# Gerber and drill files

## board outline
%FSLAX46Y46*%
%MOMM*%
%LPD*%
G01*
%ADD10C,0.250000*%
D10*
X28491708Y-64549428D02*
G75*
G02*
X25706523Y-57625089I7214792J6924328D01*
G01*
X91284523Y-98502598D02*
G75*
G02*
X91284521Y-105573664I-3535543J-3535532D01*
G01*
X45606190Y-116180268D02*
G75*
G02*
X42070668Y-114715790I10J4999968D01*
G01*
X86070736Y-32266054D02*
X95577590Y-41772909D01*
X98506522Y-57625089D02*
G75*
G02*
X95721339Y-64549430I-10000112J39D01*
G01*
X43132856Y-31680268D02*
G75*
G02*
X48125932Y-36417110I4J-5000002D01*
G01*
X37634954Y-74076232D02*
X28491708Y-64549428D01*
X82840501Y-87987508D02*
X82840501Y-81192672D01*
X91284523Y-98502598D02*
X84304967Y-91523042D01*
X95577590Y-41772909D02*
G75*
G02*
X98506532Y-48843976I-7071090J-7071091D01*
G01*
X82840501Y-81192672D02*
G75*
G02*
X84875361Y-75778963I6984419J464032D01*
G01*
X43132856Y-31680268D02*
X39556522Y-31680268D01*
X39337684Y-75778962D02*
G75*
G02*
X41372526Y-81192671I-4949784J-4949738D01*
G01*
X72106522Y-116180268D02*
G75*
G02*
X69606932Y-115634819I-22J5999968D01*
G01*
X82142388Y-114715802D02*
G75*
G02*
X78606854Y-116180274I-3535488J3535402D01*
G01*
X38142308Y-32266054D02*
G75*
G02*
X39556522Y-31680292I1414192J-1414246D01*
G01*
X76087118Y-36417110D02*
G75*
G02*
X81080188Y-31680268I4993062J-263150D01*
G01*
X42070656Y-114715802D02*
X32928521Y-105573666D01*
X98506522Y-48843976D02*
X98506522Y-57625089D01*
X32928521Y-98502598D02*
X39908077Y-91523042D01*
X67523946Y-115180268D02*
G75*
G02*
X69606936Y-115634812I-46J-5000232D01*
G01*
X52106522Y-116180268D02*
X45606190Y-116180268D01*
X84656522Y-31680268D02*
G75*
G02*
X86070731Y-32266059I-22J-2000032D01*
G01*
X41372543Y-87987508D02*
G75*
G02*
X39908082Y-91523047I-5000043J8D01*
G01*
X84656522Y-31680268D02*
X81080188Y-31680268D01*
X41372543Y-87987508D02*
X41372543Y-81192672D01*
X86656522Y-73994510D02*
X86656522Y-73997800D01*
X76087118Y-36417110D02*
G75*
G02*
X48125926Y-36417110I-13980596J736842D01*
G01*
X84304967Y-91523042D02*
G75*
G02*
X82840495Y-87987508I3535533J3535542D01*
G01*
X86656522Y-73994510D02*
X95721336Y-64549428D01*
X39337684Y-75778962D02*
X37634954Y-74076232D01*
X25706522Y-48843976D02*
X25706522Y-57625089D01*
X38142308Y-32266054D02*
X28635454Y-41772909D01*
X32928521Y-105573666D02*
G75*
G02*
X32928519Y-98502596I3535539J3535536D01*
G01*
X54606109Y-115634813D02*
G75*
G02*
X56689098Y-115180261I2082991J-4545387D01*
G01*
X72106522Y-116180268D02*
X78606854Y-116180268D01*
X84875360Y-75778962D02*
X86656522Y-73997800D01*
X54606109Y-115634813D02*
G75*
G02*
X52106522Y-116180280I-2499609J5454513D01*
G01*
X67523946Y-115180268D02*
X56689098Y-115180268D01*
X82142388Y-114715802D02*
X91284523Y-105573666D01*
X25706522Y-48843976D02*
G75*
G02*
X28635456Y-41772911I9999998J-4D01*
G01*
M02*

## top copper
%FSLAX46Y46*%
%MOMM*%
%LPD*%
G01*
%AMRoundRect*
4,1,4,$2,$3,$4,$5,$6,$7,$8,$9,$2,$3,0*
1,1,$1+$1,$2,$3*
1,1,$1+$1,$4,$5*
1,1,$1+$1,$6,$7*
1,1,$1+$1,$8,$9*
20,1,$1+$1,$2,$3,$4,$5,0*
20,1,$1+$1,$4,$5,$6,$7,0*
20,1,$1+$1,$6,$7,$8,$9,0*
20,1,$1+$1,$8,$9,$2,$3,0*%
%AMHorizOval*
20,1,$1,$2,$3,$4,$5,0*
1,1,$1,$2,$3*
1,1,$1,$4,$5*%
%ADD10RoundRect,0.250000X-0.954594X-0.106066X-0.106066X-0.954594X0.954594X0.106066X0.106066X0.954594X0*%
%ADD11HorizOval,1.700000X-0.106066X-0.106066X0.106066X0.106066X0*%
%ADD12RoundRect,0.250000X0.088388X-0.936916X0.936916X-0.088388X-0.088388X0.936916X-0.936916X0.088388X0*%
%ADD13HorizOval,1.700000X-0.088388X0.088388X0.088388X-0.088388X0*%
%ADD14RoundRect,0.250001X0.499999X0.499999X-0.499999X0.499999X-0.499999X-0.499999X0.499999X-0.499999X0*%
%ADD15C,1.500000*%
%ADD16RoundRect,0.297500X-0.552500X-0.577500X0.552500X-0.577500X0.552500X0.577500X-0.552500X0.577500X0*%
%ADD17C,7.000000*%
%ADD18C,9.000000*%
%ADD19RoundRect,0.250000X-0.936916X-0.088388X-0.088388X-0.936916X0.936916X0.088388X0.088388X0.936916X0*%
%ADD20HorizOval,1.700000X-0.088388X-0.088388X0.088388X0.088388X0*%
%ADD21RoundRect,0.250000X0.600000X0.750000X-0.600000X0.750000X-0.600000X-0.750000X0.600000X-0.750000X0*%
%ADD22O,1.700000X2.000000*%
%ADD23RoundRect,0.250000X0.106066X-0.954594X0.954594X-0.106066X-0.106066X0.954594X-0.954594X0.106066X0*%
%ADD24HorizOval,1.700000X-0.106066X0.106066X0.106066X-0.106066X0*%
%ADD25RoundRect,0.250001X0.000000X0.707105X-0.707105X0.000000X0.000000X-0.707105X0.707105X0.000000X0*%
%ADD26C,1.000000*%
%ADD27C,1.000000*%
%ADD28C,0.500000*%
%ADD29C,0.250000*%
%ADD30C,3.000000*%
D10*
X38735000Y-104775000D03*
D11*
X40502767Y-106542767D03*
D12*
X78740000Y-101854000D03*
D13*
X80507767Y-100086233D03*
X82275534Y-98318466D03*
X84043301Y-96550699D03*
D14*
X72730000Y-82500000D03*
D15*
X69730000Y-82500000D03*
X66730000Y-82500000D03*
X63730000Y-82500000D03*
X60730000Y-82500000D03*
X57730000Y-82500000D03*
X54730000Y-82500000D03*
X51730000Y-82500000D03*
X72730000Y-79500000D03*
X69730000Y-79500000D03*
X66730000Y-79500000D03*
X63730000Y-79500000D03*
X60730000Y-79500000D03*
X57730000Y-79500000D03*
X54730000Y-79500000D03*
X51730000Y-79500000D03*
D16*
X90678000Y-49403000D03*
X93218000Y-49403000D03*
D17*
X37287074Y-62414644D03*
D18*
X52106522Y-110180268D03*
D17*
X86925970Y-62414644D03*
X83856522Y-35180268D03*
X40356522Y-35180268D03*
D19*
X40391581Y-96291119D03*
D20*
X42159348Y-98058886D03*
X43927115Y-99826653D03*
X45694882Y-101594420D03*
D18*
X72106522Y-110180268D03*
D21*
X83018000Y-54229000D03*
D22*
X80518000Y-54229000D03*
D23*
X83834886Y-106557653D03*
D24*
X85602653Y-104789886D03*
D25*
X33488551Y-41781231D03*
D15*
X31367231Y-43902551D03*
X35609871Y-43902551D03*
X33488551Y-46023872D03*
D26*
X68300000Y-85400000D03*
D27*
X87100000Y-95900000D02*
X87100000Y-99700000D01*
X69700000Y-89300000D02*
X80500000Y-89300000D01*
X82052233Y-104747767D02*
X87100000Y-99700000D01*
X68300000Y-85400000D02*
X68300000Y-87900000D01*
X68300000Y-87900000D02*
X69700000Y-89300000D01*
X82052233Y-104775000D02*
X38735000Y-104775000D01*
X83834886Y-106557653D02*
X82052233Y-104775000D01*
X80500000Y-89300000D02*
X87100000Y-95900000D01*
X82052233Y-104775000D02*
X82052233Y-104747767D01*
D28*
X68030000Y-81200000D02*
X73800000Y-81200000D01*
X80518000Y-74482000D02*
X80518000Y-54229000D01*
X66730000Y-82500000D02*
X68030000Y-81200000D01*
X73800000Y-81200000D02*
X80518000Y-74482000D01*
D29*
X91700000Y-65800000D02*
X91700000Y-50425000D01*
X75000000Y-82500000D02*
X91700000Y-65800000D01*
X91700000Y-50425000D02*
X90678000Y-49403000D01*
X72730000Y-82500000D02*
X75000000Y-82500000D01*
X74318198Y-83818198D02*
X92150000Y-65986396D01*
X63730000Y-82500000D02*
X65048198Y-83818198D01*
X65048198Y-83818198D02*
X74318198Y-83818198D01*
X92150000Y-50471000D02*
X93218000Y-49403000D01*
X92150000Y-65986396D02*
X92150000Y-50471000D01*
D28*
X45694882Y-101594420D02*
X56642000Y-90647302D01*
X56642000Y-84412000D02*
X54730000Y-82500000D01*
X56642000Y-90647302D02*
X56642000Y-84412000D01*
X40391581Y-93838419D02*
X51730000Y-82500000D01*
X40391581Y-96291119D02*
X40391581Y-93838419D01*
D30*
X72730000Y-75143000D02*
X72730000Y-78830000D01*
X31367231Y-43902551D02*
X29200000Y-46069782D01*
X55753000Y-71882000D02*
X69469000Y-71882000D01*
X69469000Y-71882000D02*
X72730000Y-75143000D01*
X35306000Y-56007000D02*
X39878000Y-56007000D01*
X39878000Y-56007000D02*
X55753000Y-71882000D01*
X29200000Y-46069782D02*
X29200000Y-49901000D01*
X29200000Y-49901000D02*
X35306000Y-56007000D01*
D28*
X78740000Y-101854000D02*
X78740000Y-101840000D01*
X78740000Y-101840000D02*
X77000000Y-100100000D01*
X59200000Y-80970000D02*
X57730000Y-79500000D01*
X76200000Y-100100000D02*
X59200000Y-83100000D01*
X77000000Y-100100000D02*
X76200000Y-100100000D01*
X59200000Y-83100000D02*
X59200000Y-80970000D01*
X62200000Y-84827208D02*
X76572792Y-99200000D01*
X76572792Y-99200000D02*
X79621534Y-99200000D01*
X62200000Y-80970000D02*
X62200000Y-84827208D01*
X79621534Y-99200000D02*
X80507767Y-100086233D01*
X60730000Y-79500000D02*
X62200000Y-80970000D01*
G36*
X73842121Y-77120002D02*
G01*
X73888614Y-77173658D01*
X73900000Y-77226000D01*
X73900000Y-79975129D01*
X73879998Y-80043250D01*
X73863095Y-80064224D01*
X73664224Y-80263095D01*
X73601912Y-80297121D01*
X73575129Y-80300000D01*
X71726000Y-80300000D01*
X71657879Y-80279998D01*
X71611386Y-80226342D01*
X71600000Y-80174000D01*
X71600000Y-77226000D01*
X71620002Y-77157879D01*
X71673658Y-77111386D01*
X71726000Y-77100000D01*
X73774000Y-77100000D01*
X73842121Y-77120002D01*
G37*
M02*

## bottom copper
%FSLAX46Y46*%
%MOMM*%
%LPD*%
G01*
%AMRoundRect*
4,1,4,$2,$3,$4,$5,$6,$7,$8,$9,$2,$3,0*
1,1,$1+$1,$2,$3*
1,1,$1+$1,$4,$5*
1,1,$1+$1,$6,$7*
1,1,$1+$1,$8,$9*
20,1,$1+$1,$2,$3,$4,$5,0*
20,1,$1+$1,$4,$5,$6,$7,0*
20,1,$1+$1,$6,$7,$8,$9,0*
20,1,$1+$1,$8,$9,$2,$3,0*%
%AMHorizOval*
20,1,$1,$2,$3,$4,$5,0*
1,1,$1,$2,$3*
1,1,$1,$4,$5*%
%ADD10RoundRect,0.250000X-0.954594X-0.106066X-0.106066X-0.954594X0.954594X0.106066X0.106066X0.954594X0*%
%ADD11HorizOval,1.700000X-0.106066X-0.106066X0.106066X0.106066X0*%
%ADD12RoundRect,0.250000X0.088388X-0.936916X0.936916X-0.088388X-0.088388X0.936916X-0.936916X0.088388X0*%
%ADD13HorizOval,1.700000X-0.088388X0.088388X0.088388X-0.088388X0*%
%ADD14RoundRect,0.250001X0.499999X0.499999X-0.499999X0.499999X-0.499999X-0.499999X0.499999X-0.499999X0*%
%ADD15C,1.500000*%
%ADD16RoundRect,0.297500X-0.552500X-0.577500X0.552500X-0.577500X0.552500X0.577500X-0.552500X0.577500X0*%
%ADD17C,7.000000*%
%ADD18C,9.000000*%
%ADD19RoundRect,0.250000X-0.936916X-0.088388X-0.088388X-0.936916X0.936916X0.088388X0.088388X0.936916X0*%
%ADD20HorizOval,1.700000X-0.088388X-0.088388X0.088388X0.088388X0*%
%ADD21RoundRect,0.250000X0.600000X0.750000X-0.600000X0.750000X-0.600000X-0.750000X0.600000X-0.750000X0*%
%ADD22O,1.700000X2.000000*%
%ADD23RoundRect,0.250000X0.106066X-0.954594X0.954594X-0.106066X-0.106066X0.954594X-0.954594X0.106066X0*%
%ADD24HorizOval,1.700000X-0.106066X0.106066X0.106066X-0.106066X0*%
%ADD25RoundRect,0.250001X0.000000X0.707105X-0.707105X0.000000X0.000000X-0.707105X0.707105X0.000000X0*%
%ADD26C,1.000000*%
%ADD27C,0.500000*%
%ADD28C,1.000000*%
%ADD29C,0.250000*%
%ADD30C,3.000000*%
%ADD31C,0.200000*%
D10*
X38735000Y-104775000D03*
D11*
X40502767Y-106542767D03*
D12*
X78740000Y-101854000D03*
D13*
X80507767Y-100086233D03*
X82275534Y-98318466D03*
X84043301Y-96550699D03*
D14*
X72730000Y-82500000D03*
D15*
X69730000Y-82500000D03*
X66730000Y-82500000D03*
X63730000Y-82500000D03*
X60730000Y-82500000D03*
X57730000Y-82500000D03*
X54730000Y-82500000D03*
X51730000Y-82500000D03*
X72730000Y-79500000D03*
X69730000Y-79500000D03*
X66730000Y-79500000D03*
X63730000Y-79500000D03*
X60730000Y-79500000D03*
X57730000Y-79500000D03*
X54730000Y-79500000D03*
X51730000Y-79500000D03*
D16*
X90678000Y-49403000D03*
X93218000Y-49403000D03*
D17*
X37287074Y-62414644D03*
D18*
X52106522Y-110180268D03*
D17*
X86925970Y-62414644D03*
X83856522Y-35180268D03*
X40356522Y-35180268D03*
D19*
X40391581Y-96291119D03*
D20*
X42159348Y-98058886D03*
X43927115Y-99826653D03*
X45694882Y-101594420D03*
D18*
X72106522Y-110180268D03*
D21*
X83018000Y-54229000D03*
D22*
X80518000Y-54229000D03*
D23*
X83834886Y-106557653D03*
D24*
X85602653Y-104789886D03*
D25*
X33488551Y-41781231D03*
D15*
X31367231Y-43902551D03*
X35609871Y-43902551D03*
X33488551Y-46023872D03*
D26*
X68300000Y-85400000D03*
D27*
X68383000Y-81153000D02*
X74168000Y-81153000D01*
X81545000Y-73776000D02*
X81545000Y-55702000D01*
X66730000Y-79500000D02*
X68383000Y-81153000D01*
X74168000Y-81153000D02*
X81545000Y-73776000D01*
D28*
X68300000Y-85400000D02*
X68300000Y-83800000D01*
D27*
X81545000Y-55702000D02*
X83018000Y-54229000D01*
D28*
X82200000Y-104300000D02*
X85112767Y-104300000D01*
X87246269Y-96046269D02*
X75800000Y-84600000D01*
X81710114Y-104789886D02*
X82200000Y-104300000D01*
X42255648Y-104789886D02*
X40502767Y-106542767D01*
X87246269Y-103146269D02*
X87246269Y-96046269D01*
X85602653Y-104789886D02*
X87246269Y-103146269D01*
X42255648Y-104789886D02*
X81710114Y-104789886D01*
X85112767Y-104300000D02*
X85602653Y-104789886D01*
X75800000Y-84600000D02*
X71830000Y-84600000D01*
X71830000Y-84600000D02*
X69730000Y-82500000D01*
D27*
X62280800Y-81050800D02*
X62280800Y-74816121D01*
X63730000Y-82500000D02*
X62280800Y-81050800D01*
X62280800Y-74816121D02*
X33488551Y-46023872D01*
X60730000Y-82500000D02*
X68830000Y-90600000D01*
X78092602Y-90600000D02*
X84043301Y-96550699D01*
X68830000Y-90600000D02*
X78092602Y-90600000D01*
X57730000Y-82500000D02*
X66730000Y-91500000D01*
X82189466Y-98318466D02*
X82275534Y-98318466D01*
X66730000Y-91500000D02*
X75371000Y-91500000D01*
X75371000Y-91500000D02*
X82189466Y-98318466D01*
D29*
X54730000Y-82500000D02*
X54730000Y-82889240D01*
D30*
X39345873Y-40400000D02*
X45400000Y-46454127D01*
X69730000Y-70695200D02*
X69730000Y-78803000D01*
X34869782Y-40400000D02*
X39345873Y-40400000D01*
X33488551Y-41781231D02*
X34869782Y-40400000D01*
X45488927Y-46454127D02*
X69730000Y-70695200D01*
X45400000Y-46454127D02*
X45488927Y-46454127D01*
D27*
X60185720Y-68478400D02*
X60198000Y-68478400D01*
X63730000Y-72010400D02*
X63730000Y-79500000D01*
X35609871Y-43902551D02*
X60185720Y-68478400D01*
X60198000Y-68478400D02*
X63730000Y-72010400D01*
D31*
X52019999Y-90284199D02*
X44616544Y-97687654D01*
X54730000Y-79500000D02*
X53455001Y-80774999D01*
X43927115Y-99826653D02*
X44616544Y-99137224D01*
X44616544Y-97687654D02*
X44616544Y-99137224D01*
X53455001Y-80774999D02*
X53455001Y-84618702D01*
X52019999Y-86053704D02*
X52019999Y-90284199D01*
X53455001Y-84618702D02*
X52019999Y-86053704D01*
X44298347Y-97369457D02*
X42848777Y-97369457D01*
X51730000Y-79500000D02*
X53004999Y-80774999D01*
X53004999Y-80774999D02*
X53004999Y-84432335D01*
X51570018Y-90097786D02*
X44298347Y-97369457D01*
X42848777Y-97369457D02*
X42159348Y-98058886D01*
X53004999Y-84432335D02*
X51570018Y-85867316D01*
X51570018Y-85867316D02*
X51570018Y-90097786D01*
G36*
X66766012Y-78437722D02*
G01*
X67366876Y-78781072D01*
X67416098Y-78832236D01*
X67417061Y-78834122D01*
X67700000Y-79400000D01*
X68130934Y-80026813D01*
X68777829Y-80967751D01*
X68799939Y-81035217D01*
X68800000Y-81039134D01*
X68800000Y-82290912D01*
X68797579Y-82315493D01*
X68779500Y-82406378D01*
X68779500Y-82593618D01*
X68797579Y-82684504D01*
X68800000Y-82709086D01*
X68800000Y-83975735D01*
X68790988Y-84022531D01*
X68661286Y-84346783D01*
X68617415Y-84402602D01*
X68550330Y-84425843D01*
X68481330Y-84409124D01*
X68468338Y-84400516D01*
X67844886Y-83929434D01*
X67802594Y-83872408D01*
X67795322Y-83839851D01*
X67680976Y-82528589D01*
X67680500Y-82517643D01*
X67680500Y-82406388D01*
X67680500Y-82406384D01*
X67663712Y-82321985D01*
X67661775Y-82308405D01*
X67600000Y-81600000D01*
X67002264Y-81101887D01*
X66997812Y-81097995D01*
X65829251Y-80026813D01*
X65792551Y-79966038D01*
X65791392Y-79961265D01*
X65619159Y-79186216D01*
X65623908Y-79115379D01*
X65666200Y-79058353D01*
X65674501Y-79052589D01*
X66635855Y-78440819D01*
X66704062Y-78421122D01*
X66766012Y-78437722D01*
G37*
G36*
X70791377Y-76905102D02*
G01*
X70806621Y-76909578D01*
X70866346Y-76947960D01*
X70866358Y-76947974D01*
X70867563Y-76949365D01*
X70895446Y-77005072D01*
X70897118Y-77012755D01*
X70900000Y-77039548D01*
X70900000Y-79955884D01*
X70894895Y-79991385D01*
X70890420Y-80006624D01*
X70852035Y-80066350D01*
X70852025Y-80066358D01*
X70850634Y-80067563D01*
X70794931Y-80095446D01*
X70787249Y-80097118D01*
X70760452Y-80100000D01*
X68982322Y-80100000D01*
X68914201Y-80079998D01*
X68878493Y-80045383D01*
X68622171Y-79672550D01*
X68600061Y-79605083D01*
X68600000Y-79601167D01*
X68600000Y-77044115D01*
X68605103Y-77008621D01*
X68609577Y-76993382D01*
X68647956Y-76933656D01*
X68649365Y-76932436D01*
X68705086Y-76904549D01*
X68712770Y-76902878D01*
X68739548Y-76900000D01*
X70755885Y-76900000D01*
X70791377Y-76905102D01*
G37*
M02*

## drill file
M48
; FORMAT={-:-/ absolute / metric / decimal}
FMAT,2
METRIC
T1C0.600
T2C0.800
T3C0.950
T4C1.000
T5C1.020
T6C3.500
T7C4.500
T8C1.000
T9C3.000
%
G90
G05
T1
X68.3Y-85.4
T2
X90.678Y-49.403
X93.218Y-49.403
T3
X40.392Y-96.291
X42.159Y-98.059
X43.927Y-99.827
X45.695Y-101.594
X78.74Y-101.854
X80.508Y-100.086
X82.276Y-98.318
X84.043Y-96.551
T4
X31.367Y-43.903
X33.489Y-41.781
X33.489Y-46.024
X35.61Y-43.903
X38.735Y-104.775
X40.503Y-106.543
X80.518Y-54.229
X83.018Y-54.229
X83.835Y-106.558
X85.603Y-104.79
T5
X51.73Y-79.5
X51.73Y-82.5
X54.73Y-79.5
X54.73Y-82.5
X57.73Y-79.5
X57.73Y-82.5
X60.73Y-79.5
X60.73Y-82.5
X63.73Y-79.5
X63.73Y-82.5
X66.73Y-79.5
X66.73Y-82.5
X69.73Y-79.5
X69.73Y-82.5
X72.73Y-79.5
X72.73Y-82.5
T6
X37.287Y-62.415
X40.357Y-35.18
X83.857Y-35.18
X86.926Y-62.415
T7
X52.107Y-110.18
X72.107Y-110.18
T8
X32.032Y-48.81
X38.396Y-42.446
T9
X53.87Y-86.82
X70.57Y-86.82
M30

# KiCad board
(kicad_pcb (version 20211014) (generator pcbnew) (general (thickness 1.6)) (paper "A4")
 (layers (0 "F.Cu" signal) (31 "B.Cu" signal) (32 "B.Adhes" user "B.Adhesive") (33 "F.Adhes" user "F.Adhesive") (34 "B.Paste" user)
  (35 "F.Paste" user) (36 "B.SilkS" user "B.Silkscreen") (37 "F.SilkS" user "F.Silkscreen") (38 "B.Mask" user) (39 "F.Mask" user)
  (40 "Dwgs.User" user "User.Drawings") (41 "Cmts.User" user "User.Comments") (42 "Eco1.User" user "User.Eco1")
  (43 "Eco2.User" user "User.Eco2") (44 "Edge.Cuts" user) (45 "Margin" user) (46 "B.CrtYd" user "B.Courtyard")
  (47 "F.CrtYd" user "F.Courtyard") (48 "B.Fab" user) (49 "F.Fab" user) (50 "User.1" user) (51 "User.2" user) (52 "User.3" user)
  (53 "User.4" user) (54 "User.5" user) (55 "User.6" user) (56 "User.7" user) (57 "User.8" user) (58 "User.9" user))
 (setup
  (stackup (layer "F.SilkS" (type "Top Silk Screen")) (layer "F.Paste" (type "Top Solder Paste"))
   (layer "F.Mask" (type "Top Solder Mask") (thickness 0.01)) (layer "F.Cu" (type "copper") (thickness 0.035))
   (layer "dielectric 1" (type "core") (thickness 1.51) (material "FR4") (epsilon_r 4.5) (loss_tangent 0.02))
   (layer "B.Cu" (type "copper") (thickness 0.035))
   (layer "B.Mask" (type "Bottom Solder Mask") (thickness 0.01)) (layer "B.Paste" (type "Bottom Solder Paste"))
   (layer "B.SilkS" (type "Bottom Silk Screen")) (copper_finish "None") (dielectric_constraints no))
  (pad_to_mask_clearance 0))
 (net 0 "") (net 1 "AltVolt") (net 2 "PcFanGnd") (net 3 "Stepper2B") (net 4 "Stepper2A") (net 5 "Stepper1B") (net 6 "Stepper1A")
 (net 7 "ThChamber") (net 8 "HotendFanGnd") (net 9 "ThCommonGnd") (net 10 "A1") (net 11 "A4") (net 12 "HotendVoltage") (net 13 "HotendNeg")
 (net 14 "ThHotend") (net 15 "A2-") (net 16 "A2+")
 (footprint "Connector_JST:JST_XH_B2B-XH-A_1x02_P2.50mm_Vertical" (layer "F.Cu") (at 38.735 104.775 -45)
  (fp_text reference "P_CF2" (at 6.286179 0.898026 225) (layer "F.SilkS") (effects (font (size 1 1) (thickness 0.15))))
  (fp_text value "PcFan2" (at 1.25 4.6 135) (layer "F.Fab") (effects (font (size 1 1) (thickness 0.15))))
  (pad "1" thru_hole roundrect (at 0 0 315) (size 1.7 2) (drill 1) (layers *.Cu *.Mask) (roundrect_rratio 0.1470588235) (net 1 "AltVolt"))
  (pad "2" thru_hole oval (at 2.5 0 315) (size 1.7 2) (drill 1) (layers *.Cu *.Mask) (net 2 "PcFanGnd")))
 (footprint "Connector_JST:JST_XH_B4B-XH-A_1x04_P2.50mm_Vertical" (layer "F.Cu") (at 78.74 101.854 45)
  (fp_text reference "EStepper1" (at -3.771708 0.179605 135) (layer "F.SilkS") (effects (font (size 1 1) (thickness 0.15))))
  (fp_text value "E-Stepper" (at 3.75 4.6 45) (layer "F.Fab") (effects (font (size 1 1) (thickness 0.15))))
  (pad "1" thru_hole roundrect (at 0 0 45) (size 1.7 1.95) (drill 0.95) (layers *.Cu *.Mask) (roundrect_rratio 0.1470588235)
   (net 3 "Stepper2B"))
  (pad "2" thru_hole oval (at 2.5 0 45) (size 1.7 1.95) (drill 0.95) (layers *.Cu *.Mask) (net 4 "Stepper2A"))
  (pad "3" thru_hole oval (at 5 0 45) (size 1.7 1.95) (drill 0.95) (layers *.Cu *.Mask) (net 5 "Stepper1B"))
  (pad "4" thru_hole oval (at 7.5 0 45) (size 1.7 1.95) (drill 0.95) (layers *.Cu *.Mask) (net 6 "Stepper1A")))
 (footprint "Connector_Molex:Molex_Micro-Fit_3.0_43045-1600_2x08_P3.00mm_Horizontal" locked (layer "F.Cu") (at 72.73 82.5 180)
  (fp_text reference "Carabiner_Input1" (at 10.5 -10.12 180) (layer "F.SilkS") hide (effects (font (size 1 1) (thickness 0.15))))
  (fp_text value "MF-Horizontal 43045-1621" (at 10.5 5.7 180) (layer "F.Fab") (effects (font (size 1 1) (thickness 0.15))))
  (pad "" np_thru_hole circle locked (at 2.16 -4.32 180) (size 3 3) (drill 3) (layers *.Cu *.Mask))
  (pad "" np_thru_hole circle locked (at 18.86 -4.32 180) (size 3 3) (drill 3) (layers *.Cu *.Mask))
  (pad "1" thru_hole roundrect locked (at 0 0 180) (size 1.5 1.5) (drill 1.02) (layers *.Cu *.Mask) (roundrect_rratio 0.1666673333)
   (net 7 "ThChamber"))
  (pad "2" thru_hole circle locked (at 3 0 180) (size 1.5 1.5) (drill 1.02) (layers *.Cu *.Mask) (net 2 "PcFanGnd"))
  (pad "3" thru_hole circle locked (at 6 0 180) (size 1.5 1.5) (drill 1.02) (layers *.Cu *.Mask) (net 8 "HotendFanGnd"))
  (pad "4" thru_hole circle locked (at 9 0 180) (size 1.5 1.5) (drill 1.02) (layers *.Cu *.Mask) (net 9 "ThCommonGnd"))
  (pad "5" thru_hole circle locked (at 12 0 180) (size 1.5 1.5) (drill 1.02) (layers *.Cu *.Mask) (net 6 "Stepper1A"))
  (pad "6" thru_hole circle locked (at 15 0 180) (size 1.5 1.5) (drill 1.02) (layers *.Cu *.Mask) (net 5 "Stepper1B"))
  (pad "7" thru_hole circle locked (at 18 0 180) (size 1.5 1.5) (drill 1.02) (layers *.Cu *.Mask) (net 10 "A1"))
  (pad "8" thru_hole circle locked (at 21 0 180) (size 1.5 1.5) (drill 1.02) (layers *.Cu *.Mask) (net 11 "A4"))
  (pad "9" thru_hole circle locked (at 0 3 180) (size 1.5 1.5) (drill 1.02) (layers *.Cu *.Mask) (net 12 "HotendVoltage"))
  (pad "10" thru_hole circle locked (at 3 3 180) (size 1.5 1.5) (drill 1.02) (layers *.Cu *.Mask) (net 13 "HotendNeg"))
  (pad "11" thru_hole circle locked (at 6 3 180) (size 1.5 1.5) (drill 1.02) (layers *.Cu *.Mask) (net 1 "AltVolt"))
  (pad "12" thru_hole circle locked (at 9 3 180) (size 1.5 1.5) (drill 1.02) (layers *.Cu *.Mask) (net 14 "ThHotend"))
  (pad "13" thru_hole circle locked (at 12 3 180) (size 1.5 1.5) (drill 1.02) (layers *.Cu *.Mask) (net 4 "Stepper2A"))
  (pad "14" thru_hole circle locked (at 15 3 180) (size 1.5 1.5) (drill 1.02) (layers *.Cu *.Mask) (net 3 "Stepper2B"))
  (pad "15" thru_hole circle locked (at 18 3 180) (size 1.5 1.5) (drill 1.02) (layers *.Cu *.Mask) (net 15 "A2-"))
  (pad "16" thru_hole circle locked (at 21 3 180) (size 1.5 1.5) (drill 1.02) (layers *.Cu *.Mask) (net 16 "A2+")))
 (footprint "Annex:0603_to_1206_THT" (layer "F.Cu") (at 91.948 49.403)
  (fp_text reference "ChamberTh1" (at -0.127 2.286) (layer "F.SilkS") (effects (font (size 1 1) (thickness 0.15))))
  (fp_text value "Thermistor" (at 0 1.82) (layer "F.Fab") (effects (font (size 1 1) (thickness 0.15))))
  (pad "1" thru_hole roundrect locked (at -1.27 0) (size 1.7 1.75) (drill 0.8) (layers *.Cu *.Mask) (roundrect_rratio 0.175)
   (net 7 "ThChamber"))
  (pad "2" thru_hole roundrect locked (at 1.27 0) (size 1.7 1.75) (drill 0.8) (layers *.Cu *.Mask) (roundrect_rratio 0.175)
   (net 9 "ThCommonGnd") (die_length 12)))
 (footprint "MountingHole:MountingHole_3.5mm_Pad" (layer "F.Cu") (at 37.287074 62.414644)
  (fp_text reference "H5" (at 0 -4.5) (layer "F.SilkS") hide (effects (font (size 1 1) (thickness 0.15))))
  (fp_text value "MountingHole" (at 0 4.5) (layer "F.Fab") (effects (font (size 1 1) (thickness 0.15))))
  (pad "1" thru_hole circle (at 0 0) (size 7 7) (drill 3.5) (layers *.Cu *.Mask)))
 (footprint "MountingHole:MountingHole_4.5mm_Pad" (layer "F.Cu") (at 52.106522 110.180268)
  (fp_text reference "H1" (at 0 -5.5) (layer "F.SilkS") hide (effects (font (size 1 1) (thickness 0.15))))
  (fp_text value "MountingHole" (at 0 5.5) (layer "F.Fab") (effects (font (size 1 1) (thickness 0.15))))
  (pad "1" thru_hole circle (at 0 0) (size 9 9) (drill 4.5) (layers *.Cu *.Mask)))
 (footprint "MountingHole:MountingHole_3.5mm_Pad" (layer "F.Cu") (at 86.92597 62.414644)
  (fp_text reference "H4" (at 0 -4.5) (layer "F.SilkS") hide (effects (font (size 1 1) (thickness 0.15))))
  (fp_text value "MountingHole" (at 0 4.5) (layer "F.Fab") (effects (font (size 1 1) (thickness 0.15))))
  (pad "1" thru_hole circle (at 0 0) (size 7 7) (drill 3.5) (layers *.Cu *.Mask)))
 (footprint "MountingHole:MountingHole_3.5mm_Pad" (layer "F.Cu") (at 83.856522 35.180268)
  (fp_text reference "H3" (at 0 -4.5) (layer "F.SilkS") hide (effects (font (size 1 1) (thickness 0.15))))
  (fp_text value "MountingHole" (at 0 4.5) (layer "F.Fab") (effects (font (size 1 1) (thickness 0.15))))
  (pad "1" thru_hole circle (at 0 0) (size 7 7) (drill 3.5) (layers *.Cu *.Mask)))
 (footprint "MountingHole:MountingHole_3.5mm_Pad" (layer "F.Cu") (at 40.356522 35.180268)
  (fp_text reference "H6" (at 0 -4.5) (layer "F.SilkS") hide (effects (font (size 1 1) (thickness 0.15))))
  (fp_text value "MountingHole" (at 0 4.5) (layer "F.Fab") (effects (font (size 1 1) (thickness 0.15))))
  (pad "1" thru_hole circle (at 0 0) (size 7 7) (drill 3.5) (layers *.Cu *.Mask)))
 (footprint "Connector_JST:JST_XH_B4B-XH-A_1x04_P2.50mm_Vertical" (layer "F.Cu") (at 40.391581 96.291119 -45)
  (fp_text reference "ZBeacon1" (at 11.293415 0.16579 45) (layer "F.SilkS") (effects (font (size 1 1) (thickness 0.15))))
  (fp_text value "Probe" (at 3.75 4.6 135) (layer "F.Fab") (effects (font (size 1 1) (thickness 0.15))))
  (pad "1" thru_hole roundrect (at 0 0 315) (size 1.7 1.95) (drill 0.95) (layers *.Cu *.Mask) (roundrect_rratio 0.1470588235) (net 11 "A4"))
  (pad "2" thru_hole oval (at 2.5 0 315) (size 1.7 1.95) (drill 0.95) (layers *.Cu *.Mask) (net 16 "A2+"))
  (pad "3" thru_hole oval (at 5 0 315) (size 1.7 1.95) (drill 0.95) (layers *.Cu *.Mask) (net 15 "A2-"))
  (pad "4" thru_hole oval (at 7.5 0 315) (size 1.7 1.95) (drill 0.95) (layers *.Cu *.Mask) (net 10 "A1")))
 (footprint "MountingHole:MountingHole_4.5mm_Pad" (layer "F.Cu") (at 72.106522 110.180268)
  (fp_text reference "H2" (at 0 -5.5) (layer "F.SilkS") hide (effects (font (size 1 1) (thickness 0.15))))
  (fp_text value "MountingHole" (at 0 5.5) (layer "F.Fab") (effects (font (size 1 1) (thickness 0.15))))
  (pad "1" thru_hole circle (at 0 0) (size 9 9) (drill 4.5) (layers *.Cu *.Mask)))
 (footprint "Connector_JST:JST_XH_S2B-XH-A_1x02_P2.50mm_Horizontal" (layer "F.Cu") (at 83.018 54.229 180)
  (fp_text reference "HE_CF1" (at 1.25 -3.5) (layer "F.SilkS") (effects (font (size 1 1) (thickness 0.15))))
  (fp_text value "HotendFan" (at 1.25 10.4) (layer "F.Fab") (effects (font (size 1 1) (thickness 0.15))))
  (pad "1" thru_hole roundrect (at 0 0 180) (size 1.7 2) (drill 1) (layers *.Cu *.Mask) (roundrect_rratio 0.1470588235) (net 1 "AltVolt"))
  (pad "2" thru_hole oval (at 2.5 0 180) (size 1.7 2) (drill 1) (layers *.Cu *.Mask) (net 8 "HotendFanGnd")))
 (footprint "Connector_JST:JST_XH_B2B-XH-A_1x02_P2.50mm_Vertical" (layer "F.Cu") (at 83.834886 106.557653 45)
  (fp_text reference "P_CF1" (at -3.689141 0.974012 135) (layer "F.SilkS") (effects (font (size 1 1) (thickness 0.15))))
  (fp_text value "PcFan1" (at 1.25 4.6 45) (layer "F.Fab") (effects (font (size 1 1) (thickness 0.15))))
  (pad "1" thru_hole roundrect (at 0 0 45) (size 1.7 2) (drill 1) (layers *.Cu *.Mask) (roundrect_rratio 0.1470588235) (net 1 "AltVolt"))
  (pad "2" thru_hole oval (at 2.5 0 45) (size 1.7 2) (drill 1) (layers *.Cu *.Mask) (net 2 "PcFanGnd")))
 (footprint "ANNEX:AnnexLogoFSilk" (layer "F.Cu") (at 91.948 44.196)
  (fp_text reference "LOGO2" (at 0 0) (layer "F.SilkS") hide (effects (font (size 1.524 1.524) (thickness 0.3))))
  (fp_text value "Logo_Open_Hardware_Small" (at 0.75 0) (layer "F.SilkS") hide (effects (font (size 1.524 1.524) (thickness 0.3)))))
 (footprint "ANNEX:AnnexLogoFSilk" (layer "B.Cu") (at 91.694 44.196 180)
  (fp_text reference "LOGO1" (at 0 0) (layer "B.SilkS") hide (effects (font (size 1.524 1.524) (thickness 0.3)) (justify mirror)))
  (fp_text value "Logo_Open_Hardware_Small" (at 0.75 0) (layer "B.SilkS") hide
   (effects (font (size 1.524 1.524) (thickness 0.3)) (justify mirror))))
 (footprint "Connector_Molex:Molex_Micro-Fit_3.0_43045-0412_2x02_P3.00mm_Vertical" (layer "B.Cu") (at 33.488551 41.781231 -135)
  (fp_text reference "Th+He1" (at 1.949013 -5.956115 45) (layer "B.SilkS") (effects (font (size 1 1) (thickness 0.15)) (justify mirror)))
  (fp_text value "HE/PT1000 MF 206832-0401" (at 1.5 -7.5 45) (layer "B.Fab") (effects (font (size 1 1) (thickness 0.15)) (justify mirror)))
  (pad "" np_thru_hole circle (at 6 -3.94 225) (size 1 1) (drill 1) (layers *.Cu *.Mask))
  (pad "" np_thru_hole circle (at -3 -3.94 225) (size 1 1) (drill 1) (layers *.Cu *.Mask))
  (pad "1" thru_hole roundrect (at 0 0 225) (size 1.5 1.5) (drill 1) (layers *.Cu *.Mask) (roundrect_rratio 0.1666673333)
   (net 13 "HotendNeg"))
  (pad "2" thru_hole circle (at 3 0 225) (size 1.5 1.5) (drill 1) (layers *.Cu *.Mask) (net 12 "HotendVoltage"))
  (pad "3" thru_hole circle (at 0 -3 225) (size 1.5 1.5) (drill 1) (layers *.Cu *.Mask) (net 14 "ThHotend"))
  (pad "4" thru_hole circle (at 3 -3 225) (size 1.5 1.5) (drill 1) (layers *.Cu *.Mask) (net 9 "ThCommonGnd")))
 (gr_arc (start 28.491708 64.549428) (mid 26.428911 61.356836) (end 25.706522 57.625089) (layer "Edge.Cuts") (width 0.25))
 (gr_arc (start 91.284523 98.502598) (mid 92.748987 102.038131) (end 91.284523 105.573666) (layer "Edge.Cuts") (width 0.25))
 (gr_arc (start 45.60619 116.180268) (mid 43.692773 115.799666) (end 42.070656 114.715802) (layer "Edge.Cuts") (width 0.25))
 (gr_line (start 86.070736 32.266054) (end 95.57759 41.772909) (layer "Edge.Cuts") (width 0.25))
 (gr_arc (start 98.506522 57.625089) (mid 97.784126 61.356831) (end 95.721336 64.549428) (layer "Edge.Cuts") (width 0.25))
 (gr_arc (start 43.132856 31.680268) (mid 46.574092 33.052887) (end 48.125926 36.41711) (layer "Edge.Cuts") (width 0.25))
 (gr_line (start 37.634954 74.076232) (end 28.491708 64.549428) (layer "Edge.Cuts") (width 0.25))
 (gr_line (start 82.840501 87.987508) (end 82.840501 81.192672) (layer "Edge.Cuts") (width 0.25))
 (gr_line (start 91.284523 98.502598) (end 84.304967 91.523042) (layer "Edge.Cuts") (width 0.25))
 (gr_arc (start 95.57759 41.772909) (mid 97.745314 45.017143) (end 98.506522 48.843976) (layer "Edge.Cuts") (width 0.25))
 (gr_arc (start 82.840501 81.192672) (mid 83.272668 78.265829) (end 84.87536 75.778962) (layer "Edge.Cuts") (width 0.25))
 (gr_line (start 43.132856 31.680268) (end 39.556522 31.680268) (layer "Edge.Cuts") (width 0.25))
 (gr_arc (start 39.337684 75.778962) (mid 40.940361 78.265839) (end 41.372543 81.192672) (layer "Edge.Cuts") (width 0.25))
 (gr_arc (start 72.106522 116.180268) (mid 70.827317 116.042318) (end 69.606935 115.634813) (layer "Edge.Cuts") (width 0.25))
 (gr_arc (start 82.142388 114.715802) (mid 80.520273 115.799676) (end 78.606854 116.180268) (layer "Edge.Cuts") (width 0.25))
 (gr_arc (start 38.142308 32.266054) (mid 38.791155 31.832509) (end 39.556522 31.680268) (layer "Edge.Cuts") (width 0.25))
 (gr_arc (start 76.087118 36.41711) (mid 77.638952 33.052885) (end 81.080188 31.680268) (layer "Edge.Cuts") (width 0.25))
 (gr_line (start 42.070656 114.715802) (end 32.928521 105.573666) (layer "Edge.Cuts") (width 0.25))
 (gr_line (start 98.506522 48.843976) (end 98.506522 57.625089) (layer "Edge.Cuts") (width 0.25))
 (gr_line (start 32.928521 98.502598) (end 39.908077 91.523042) (layer "Edge.Cuts") (width 0.25))
 (gr_arc (start 67.523946 115.180268) (mid 68.589948 115.295231) (end 69.606935 115.634813) (layer "Edge.Cuts") (width 0.25))
 (gr_line (start 52.106522 116.180268) (end 45.60619 116.180268) (layer "Edge.Cuts") (width 0.25))
 (gr_arc (start 84.656522 31.680268) (mid 85.421889 31.832509) (end 86.070736 32.266054) (layer "Edge.Cuts") (width 0.25))
 (gr_arc (start 41.372543 87.987508) (mid 40.991941 89.900925) (end 39.908077 91.523042) (layer "Edge.Cuts") (width 0.25))
 (gr_line (start 84.656522 31.680268) (end 81.080188 31.680268) (layer "Edge.Cuts") (width 0.25))
 (gr_line (start 41.372543 87.987508) (end 41.372543 81.192672) (layer "Edge.Cuts") (width 0.25))
 (gr_line (start 86.656522 73.99451) (end 86.656522 73.9978) (layer "Edge.Cuts") (width 0.25))
 (gr_arc (start 76.087118 36.41711) (mid 62.106522 49.680268) (end 48.125926 36.41711) (layer "Edge.Cuts") (width 0.25))
 (gr_arc (start 84.304967 91.523042) (mid 83.221103 89.900925) (end 82.840501 87.987508) (layer "Edge.Cuts") (width 0.25))
 (gr_line (start 86.656522 73.99451) (end 95.721336 64.549428) (layer "Edge.Cuts") (width 0.25))
 (gr_line (start 39.337684 75.778962) (end 37.634954 74.076232) (layer "Edge.Cuts") (width 0.25))
 (gr_line (start 25.706522 48.843976) (end 25.706522 57.625089) (layer "Edge.Cuts") (width 0.25))
 (gr_line (start 38.142308 32.266054) (end 28.635454 41.772909) (layer "Edge.Cuts") (width 0.25))
 (gr_arc (start 32.928521 105.573666) (mid 31.464055 102.038132) (end 32.928521 98.502598) (layer "Edge.Cuts") (width 0.25))
 (gr_arc (start 54.606109 115.634813) (mid 55.623094 115.295225) (end 56.689098 115.180268) (layer "Edge.Cuts") (width 0.25))
 (gr_line (start 72.106522 116.180268) (end 78.606854 116.180268) (layer "Edge.Cuts") (width 0.25))
 (gr_line (start 84.87536 75.778962) (end 86.656522 73.9978) (layer "Edge.Cuts") (width 0.25))
 (gr_arc (start 54.606109 115.634813) (mid 53.385726 116.042318) (end 52.106522 116.180268) (layer "Edge.Cuts") (width 0.25))
 (gr_line (start 67.523946 115.180268) (end 56.689098 115.180268) (layer "Edge.Cuts") (width 0.25))
 (gr_line (start 82.142388 114.715802) (end 91.284523 105.573666) (layer "Edge.Cuts") (width 0.25))
 (gr_arc (start 25.706522 48.843976) (mid 26.467727 45.017142) (end 28.635454 41.772909) (layer "Edge.Cuts") (width 0.25))
 (segment (start 87.1 95.9) (end 87.1 99.7) (width 1) (layer "F.Cu") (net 1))
 (segment (start 69.7 89.3) (end 80.5 89.3) (width 1) (layer "F.Cu") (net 1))
 (segment (start 82.052233 104.747767) (end 87.1 99.7) (width 1) (layer "F.Cu") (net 1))
 (segment (start 68.3 85.4) (end 68.3 87.9) (width 1) (layer "F.Cu") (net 1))
 (segment (start 68.3 87.9) (end 69.7 89.3) (width 1) (layer "F.Cu") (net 1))
 (segment (start 82.052233 104.775) (end 38.735 104.775) (width 1) (layer "F.Cu") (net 1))
 (segment (start 83.834886 106.557653) (end 82.052233 104.775) (width 1) (layer "F.Cu") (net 1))
 (segment (start 80.5 89.3) (end 87.1 95.9) (width 1) (layer "F.Cu") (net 1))
 (segment (start 82.052233 104.775) (end 82.052233 104.747767) (width 1) (layer "F.Cu") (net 1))
 (via (at 68.3 85.4) (size 1) (drill 0.6) (layers "F.Cu" "B.Cu") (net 1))
 (segment (start 68.383 81.153) (end 74.168 81.153) (width 0.5) (layer "B.Cu") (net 1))
 (segment (start 81.545 73.776) (end 81.545 55.702) (width 0.5) (layer "B.Cu") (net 1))
 (segment (start 66.73 79.5) (end 68.383 81.153) (width 0.5) (layer "B.Cu") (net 1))
 (segment (start 74.168 81.153) (end 81.545 73.776) (width 0.5) (layer "B.Cu") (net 1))
 (segment (start 68.3 85.4) (end 68.3 83.8) (width 1) (layer "B.Cu") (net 1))
 (segment (start 81.545 55.702) (end 83.018 54.229) (width 0.5) (layer "B.Cu") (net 1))
 (segment (start 68.03 81.2) (end 73.8 81.2) (width 0.5) (layer "F.Cu") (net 8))
 (segment (start 80.518 74.482) (end 80.518 54.229) (width 0.5) (layer "F.Cu") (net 8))
 (segment (start 66.73 82.5) (end 68.03 81.2) (width 0.5) (layer "F.Cu") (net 8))
 (segment (start 73.8 81.2) (end 80.518 74.482) (width 0.5) (layer "F.Cu") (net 8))
 (segment (start 91.7 65.8) (end 91.7 50.425) (width 0.25) (layer "F.Cu") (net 7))
 (segment (start 75 82.5) (end 91.7 65.8) (width 0.25) (layer "F.Cu") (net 7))
 (segment (start 91.7 50.425) (end 90.678 49.403) (width 0.25) (layer "F.Cu") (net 7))
 (segment (start 72.73 82.5) (end 75 82.5) (width 0.25) (layer "F.Cu") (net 7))
 (segment (start 82.2 104.3) (end 85.112767 104.3) (width 1) (layer "B.Cu") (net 2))
 (segment (start 87.246269 96.046269) (end 75.8 84.6) (width 1) (layer "B.Cu") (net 2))
 (segment (start 81.710114 104.789886) (end 82.2 104.3) (width 1) (layer "B.Cu") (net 2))
 (segment (start 42.255648 104.789886) (end 40.502767 106.542767) (width 1) (layer "B.Cu") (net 2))
 (segment (start 87.246269 103.146269) (end 87.246269 96.046269) (width 1) (layer "B.Cu") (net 2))
 (segment (start 85.602653 104.789886) (end 87.246269 103.146269) (width 1) (layer "B.Cu") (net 2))
 (segment (start 42.255648 104.789886) (end 81.710114 104.789886) (width 1) (layer "B.Cu") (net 2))
 (segment (start 85.112767 104.3) (end 85.602653 104.789886) (width 1) (layer "B.Cu") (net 2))
 (segment (start 75.8 84.6) (end 71.83 84.6) (width 1) (layer "B.Cu") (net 2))
 (segment (start 71.83 84.6) (end 69.73 82.5) (width 1) (layer "B.Cu") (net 2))
 (segment (start 74.318198 83.818198) (end 92.15 65.986396) (width 0.25) (layer "F.Cu") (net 9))
 (segment (start 63.73 82.5) (end 65.048198 83.818198) (width 0.25) (layer "F.Cu") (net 9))
 (segment (start 65.048198 83.818198) (end 74.318198 83.818198) (width 0.25) (layer "F.Cu") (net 9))
 (segment (start 92.15 50.471) (end 93.218 49.403) (width 0.25) (layer "F.Cu") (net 9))
 (segment (start 92.15 65.986396) (end 92.15 50.471) (width 0.25) (layer "F.Cu") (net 9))
 (segment (start 62.2808 81.0508) (end 62.2808 74.816121) (width 0.5) (layer "B.Cu") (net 9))
 (segment (start 63.73 82.5) (end 62.2808 81.0508) (width 0.5) (layer "B.Cu") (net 9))
 (segment (start 62.2808 74.816121) (end 33.488551 46.023872) (width 0.5) (layer "B.Cu") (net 9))
 (segment (start 60.73 82.5) (end 68.83 90.6) (width 0.5) (layer "B.Cu") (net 6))
 (segment (start 78.092602 90.6) (end 84.043301 96.550699) (width 0.5) (layer "B.Cu") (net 6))
 (segment (start 68.83 90.6) (end 78.092602 90.6) (width 0.5) (layer "B.Cu") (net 6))
 (segment (start 57.73 82.5) (end 66.73 91.5) (width 0.5) (layer "B.Cu") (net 5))
 (segment (start 82.189466 98.318466) (end 82.275534 98.318466) (width 0.5) (layer "B.Cu") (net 5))
 (segment (start 66.73 91.5) (end 75.371 91.5) (width 0.5) (layer "B.Cu") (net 5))
 (segment (start 75.371 91.5) (end 82.189466 98.318466) (width 0.5) (layer "B.Cu") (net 5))
 (segment (start 45.694882 101.59442) (end 56.642 90.647302) (width 0.5) (layer "F.Cu") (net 10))
 (segment (start 56.642 84.412) (end 54.73 82.5) (width 0.5) (layer "F.Cu") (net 10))
 (segment (start 56.642 90.647302) (end 56.642 84.412) (width 0.5) (layer "F.Cu") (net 10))
 (segment (start 54.73 82.5) (end 54.73 82.88924) (width 0.25) (layer "B.Cu") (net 10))
 (segment (start 40.391581 93.838419) (end 51.73 82.5) (width 0.5) (layer "F.Cu") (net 11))
 (segment (start 40.391581 96.291119) (end 40.391581 93.838419) (width 0.5) (layer "F.Cu") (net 11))
 (segment (start 72.73 75.143) (end 72.73 78.83) (width 3) (layer "F.Cu") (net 12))
 (segment (start 31.367231 43.902551) (end 29.2 46.069782) (width 3) (layer "F.Cu") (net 12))
 (segment (start 55.753 71.882) (end 69.469 71.882) (width 3) (layer "F.Cu") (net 12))
 (segment (start 69.469 71.882) (end 72.73 75.143) (width 3) (layer "F.Cu") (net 12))
 (segment (start 35.306 56.007) (end 39.878 56.007) (width 3) (layer "F.Cu") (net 12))
 (segment (start 39.878 56.007) (end 55.753 71.882) (width 3) (layer "F.Cu") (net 12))
 (segment (start 29.2 46.069782) (end 29.2 49.901) (width 3) (layer "F.Cu") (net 12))
 (segment (start 29.2 49.901) (end 35.306 56.007) (width 3) (layer "F.Cu") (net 12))
 (segment (start 39.345873 40.4) (end 45.4 46.454127) (width 3) (layer "B.Cu") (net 13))
 (segment (start 69.73 70.6952) (end 69.73 78.803) (width 3) (layer "B.Cu") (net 13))
 (segment (start 34.869782 40.4) (end 39.345873 40.4) (width 3) (layer "B.Cu") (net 13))
 (segment (start 33.488551 41.781231) (end 34.869782 40.4) (width 3) (layer "B.Cu") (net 13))
 (segment (start 45.488927 46.454127) (end 69.73 70.6952) (width 3) (layer "B.Cu") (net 13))
 (segment (start 45.4 46.454127) (end 45.488927 46.454127) (width 3) (layer "B.Cu") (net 13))
 (segment (start 60.18572 68.4784) (end 60.198 68.4784) (width 0.5) (layer "B.Cu") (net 14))
 (segment (start 63.73 72.0104) (end 63.73 79.5) (width 0.5) (layer "B.Cu") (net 14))
 (segment (start 35.609871 43.902551) (end 60.18572 68.4784) (width 0.5) (layer "B.Cu") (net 14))
 (segment (start 60.198 68.4784) (end 63.73 72.0104) (width 0.5) (layer "B.Cu") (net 14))
 (segment (start 78.74 101.854) (end 78.74 101.84) (width 0.5) (layer "F.Cu") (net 3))
 (segment (start 78.74 101.84) (end 77 100.1) (width 0.5) (layer "F.Cu") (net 3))
 (segment (start 59.2 80.97) (end 57.73 79.5) (width 0.5) (layer "F.Cu") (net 3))
 (segment (start 76.2 100.1) (end 59.2 83.1) (width 0.5) (layer "F.Cu") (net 3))
 (segment (start 77 100.1) (end 76.2 100.1) (width 0.5) (layer "F.Cu") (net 3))
 (segment (start 59.2 83.1) (end 59.2 80.97) (width 0.5) (layer "F.Cu") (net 3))
 (segment (start 62.2 84.827208) (end 76.572792 99.2) (width 0.5) (layer "F.Cu") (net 4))
 (segment (start 76.572792 99.2) (end 79.621534 99.2) (width 0.5) (layer "F.Cu") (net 4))
 (segment (start 62.2 80.97) (end 62.2 84.827208) (width 0.5) (layer "F.Cu") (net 4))
 (segment (start 79.621534 99.2) (end 80.507767 100.086233) (width 0.5) (layer "F.Cu") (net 4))
 (segment (start 60.73 79.5) (end 62.2 80.97) (width 0.5) (layer "F.Cu") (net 4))
 (segment (start 52.019999 90.284199) (end 44.616544 97.687654) (width 0.2) (layer "B.Cu") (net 15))
 (segment (start 54.73 79.5) (end 53.455001 80.774999) (width 0.2) (layer "B.Cu") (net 15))
 (segment (start 43.927115 99.826653) (end 44.616544 99.137224) (width 0.2) (layer "B.Cu") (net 15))
 (segment (start 44.616544 97.687654) (end 44.616544 99.137224) (width 0.2) (layer "B.Cu") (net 15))
 (segment (start 53.455001 80.774999) (end 53.455001 84.618702) (width 0.2) (layer "B.Cu") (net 15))
 (segment (start 52.019999 86.053704) (end 52.019999 90.284199) (width 0.2) (layer "B.Cu") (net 15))
 (segment (start 53.455001 84.618702) (end 52.019999 86.053704) (width 0.2) (layer "B.Cu") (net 15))
 (segment (start 44.298347 97.369457) (end 42.848777 97.369457) (width 0.2) (layer "B.Cu") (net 16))
 (segment (start 51.73 79.5) (end 53.004999 80.774999) (width 0.2) (layer "B.Cu") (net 16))
 (segment (start 53.004999 80.774999) (end 53.004999 84.432335) (width 0.2) (layer "B.Cu") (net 16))
 (segment (start 51.570018 90.097786) (end 44.298347 97.369457) (width 0.2) (layer "B.Cu") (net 16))
 (segment (start 42.848777 97.369457) (end 42.159348 98.058886) (width 0.2) (layer "B.Cu") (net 16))
 (segment (start 53.004999 84.432335) (end 51.570018 85.867316) (width 0.2) (layer "B.Cu") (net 16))
 (segment (start 51.570018 85.867316) (end 51.570018 90.097786) (width 0.2) (layer "B.Cu") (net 16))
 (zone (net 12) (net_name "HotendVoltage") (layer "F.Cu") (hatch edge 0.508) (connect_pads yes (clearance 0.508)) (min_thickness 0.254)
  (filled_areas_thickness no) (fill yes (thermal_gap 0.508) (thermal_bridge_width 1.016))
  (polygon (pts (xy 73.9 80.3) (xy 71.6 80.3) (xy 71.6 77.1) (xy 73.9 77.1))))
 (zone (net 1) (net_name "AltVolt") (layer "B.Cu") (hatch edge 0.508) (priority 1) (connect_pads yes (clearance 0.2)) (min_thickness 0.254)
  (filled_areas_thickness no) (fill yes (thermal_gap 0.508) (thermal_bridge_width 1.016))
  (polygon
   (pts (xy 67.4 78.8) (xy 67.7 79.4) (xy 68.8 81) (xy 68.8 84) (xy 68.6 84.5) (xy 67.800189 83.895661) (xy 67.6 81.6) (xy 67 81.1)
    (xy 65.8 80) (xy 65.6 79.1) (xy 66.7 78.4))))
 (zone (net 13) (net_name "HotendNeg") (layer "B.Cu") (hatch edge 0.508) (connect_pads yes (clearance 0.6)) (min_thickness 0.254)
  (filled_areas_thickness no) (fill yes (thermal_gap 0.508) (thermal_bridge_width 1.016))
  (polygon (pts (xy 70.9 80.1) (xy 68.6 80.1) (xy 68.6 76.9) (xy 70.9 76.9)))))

